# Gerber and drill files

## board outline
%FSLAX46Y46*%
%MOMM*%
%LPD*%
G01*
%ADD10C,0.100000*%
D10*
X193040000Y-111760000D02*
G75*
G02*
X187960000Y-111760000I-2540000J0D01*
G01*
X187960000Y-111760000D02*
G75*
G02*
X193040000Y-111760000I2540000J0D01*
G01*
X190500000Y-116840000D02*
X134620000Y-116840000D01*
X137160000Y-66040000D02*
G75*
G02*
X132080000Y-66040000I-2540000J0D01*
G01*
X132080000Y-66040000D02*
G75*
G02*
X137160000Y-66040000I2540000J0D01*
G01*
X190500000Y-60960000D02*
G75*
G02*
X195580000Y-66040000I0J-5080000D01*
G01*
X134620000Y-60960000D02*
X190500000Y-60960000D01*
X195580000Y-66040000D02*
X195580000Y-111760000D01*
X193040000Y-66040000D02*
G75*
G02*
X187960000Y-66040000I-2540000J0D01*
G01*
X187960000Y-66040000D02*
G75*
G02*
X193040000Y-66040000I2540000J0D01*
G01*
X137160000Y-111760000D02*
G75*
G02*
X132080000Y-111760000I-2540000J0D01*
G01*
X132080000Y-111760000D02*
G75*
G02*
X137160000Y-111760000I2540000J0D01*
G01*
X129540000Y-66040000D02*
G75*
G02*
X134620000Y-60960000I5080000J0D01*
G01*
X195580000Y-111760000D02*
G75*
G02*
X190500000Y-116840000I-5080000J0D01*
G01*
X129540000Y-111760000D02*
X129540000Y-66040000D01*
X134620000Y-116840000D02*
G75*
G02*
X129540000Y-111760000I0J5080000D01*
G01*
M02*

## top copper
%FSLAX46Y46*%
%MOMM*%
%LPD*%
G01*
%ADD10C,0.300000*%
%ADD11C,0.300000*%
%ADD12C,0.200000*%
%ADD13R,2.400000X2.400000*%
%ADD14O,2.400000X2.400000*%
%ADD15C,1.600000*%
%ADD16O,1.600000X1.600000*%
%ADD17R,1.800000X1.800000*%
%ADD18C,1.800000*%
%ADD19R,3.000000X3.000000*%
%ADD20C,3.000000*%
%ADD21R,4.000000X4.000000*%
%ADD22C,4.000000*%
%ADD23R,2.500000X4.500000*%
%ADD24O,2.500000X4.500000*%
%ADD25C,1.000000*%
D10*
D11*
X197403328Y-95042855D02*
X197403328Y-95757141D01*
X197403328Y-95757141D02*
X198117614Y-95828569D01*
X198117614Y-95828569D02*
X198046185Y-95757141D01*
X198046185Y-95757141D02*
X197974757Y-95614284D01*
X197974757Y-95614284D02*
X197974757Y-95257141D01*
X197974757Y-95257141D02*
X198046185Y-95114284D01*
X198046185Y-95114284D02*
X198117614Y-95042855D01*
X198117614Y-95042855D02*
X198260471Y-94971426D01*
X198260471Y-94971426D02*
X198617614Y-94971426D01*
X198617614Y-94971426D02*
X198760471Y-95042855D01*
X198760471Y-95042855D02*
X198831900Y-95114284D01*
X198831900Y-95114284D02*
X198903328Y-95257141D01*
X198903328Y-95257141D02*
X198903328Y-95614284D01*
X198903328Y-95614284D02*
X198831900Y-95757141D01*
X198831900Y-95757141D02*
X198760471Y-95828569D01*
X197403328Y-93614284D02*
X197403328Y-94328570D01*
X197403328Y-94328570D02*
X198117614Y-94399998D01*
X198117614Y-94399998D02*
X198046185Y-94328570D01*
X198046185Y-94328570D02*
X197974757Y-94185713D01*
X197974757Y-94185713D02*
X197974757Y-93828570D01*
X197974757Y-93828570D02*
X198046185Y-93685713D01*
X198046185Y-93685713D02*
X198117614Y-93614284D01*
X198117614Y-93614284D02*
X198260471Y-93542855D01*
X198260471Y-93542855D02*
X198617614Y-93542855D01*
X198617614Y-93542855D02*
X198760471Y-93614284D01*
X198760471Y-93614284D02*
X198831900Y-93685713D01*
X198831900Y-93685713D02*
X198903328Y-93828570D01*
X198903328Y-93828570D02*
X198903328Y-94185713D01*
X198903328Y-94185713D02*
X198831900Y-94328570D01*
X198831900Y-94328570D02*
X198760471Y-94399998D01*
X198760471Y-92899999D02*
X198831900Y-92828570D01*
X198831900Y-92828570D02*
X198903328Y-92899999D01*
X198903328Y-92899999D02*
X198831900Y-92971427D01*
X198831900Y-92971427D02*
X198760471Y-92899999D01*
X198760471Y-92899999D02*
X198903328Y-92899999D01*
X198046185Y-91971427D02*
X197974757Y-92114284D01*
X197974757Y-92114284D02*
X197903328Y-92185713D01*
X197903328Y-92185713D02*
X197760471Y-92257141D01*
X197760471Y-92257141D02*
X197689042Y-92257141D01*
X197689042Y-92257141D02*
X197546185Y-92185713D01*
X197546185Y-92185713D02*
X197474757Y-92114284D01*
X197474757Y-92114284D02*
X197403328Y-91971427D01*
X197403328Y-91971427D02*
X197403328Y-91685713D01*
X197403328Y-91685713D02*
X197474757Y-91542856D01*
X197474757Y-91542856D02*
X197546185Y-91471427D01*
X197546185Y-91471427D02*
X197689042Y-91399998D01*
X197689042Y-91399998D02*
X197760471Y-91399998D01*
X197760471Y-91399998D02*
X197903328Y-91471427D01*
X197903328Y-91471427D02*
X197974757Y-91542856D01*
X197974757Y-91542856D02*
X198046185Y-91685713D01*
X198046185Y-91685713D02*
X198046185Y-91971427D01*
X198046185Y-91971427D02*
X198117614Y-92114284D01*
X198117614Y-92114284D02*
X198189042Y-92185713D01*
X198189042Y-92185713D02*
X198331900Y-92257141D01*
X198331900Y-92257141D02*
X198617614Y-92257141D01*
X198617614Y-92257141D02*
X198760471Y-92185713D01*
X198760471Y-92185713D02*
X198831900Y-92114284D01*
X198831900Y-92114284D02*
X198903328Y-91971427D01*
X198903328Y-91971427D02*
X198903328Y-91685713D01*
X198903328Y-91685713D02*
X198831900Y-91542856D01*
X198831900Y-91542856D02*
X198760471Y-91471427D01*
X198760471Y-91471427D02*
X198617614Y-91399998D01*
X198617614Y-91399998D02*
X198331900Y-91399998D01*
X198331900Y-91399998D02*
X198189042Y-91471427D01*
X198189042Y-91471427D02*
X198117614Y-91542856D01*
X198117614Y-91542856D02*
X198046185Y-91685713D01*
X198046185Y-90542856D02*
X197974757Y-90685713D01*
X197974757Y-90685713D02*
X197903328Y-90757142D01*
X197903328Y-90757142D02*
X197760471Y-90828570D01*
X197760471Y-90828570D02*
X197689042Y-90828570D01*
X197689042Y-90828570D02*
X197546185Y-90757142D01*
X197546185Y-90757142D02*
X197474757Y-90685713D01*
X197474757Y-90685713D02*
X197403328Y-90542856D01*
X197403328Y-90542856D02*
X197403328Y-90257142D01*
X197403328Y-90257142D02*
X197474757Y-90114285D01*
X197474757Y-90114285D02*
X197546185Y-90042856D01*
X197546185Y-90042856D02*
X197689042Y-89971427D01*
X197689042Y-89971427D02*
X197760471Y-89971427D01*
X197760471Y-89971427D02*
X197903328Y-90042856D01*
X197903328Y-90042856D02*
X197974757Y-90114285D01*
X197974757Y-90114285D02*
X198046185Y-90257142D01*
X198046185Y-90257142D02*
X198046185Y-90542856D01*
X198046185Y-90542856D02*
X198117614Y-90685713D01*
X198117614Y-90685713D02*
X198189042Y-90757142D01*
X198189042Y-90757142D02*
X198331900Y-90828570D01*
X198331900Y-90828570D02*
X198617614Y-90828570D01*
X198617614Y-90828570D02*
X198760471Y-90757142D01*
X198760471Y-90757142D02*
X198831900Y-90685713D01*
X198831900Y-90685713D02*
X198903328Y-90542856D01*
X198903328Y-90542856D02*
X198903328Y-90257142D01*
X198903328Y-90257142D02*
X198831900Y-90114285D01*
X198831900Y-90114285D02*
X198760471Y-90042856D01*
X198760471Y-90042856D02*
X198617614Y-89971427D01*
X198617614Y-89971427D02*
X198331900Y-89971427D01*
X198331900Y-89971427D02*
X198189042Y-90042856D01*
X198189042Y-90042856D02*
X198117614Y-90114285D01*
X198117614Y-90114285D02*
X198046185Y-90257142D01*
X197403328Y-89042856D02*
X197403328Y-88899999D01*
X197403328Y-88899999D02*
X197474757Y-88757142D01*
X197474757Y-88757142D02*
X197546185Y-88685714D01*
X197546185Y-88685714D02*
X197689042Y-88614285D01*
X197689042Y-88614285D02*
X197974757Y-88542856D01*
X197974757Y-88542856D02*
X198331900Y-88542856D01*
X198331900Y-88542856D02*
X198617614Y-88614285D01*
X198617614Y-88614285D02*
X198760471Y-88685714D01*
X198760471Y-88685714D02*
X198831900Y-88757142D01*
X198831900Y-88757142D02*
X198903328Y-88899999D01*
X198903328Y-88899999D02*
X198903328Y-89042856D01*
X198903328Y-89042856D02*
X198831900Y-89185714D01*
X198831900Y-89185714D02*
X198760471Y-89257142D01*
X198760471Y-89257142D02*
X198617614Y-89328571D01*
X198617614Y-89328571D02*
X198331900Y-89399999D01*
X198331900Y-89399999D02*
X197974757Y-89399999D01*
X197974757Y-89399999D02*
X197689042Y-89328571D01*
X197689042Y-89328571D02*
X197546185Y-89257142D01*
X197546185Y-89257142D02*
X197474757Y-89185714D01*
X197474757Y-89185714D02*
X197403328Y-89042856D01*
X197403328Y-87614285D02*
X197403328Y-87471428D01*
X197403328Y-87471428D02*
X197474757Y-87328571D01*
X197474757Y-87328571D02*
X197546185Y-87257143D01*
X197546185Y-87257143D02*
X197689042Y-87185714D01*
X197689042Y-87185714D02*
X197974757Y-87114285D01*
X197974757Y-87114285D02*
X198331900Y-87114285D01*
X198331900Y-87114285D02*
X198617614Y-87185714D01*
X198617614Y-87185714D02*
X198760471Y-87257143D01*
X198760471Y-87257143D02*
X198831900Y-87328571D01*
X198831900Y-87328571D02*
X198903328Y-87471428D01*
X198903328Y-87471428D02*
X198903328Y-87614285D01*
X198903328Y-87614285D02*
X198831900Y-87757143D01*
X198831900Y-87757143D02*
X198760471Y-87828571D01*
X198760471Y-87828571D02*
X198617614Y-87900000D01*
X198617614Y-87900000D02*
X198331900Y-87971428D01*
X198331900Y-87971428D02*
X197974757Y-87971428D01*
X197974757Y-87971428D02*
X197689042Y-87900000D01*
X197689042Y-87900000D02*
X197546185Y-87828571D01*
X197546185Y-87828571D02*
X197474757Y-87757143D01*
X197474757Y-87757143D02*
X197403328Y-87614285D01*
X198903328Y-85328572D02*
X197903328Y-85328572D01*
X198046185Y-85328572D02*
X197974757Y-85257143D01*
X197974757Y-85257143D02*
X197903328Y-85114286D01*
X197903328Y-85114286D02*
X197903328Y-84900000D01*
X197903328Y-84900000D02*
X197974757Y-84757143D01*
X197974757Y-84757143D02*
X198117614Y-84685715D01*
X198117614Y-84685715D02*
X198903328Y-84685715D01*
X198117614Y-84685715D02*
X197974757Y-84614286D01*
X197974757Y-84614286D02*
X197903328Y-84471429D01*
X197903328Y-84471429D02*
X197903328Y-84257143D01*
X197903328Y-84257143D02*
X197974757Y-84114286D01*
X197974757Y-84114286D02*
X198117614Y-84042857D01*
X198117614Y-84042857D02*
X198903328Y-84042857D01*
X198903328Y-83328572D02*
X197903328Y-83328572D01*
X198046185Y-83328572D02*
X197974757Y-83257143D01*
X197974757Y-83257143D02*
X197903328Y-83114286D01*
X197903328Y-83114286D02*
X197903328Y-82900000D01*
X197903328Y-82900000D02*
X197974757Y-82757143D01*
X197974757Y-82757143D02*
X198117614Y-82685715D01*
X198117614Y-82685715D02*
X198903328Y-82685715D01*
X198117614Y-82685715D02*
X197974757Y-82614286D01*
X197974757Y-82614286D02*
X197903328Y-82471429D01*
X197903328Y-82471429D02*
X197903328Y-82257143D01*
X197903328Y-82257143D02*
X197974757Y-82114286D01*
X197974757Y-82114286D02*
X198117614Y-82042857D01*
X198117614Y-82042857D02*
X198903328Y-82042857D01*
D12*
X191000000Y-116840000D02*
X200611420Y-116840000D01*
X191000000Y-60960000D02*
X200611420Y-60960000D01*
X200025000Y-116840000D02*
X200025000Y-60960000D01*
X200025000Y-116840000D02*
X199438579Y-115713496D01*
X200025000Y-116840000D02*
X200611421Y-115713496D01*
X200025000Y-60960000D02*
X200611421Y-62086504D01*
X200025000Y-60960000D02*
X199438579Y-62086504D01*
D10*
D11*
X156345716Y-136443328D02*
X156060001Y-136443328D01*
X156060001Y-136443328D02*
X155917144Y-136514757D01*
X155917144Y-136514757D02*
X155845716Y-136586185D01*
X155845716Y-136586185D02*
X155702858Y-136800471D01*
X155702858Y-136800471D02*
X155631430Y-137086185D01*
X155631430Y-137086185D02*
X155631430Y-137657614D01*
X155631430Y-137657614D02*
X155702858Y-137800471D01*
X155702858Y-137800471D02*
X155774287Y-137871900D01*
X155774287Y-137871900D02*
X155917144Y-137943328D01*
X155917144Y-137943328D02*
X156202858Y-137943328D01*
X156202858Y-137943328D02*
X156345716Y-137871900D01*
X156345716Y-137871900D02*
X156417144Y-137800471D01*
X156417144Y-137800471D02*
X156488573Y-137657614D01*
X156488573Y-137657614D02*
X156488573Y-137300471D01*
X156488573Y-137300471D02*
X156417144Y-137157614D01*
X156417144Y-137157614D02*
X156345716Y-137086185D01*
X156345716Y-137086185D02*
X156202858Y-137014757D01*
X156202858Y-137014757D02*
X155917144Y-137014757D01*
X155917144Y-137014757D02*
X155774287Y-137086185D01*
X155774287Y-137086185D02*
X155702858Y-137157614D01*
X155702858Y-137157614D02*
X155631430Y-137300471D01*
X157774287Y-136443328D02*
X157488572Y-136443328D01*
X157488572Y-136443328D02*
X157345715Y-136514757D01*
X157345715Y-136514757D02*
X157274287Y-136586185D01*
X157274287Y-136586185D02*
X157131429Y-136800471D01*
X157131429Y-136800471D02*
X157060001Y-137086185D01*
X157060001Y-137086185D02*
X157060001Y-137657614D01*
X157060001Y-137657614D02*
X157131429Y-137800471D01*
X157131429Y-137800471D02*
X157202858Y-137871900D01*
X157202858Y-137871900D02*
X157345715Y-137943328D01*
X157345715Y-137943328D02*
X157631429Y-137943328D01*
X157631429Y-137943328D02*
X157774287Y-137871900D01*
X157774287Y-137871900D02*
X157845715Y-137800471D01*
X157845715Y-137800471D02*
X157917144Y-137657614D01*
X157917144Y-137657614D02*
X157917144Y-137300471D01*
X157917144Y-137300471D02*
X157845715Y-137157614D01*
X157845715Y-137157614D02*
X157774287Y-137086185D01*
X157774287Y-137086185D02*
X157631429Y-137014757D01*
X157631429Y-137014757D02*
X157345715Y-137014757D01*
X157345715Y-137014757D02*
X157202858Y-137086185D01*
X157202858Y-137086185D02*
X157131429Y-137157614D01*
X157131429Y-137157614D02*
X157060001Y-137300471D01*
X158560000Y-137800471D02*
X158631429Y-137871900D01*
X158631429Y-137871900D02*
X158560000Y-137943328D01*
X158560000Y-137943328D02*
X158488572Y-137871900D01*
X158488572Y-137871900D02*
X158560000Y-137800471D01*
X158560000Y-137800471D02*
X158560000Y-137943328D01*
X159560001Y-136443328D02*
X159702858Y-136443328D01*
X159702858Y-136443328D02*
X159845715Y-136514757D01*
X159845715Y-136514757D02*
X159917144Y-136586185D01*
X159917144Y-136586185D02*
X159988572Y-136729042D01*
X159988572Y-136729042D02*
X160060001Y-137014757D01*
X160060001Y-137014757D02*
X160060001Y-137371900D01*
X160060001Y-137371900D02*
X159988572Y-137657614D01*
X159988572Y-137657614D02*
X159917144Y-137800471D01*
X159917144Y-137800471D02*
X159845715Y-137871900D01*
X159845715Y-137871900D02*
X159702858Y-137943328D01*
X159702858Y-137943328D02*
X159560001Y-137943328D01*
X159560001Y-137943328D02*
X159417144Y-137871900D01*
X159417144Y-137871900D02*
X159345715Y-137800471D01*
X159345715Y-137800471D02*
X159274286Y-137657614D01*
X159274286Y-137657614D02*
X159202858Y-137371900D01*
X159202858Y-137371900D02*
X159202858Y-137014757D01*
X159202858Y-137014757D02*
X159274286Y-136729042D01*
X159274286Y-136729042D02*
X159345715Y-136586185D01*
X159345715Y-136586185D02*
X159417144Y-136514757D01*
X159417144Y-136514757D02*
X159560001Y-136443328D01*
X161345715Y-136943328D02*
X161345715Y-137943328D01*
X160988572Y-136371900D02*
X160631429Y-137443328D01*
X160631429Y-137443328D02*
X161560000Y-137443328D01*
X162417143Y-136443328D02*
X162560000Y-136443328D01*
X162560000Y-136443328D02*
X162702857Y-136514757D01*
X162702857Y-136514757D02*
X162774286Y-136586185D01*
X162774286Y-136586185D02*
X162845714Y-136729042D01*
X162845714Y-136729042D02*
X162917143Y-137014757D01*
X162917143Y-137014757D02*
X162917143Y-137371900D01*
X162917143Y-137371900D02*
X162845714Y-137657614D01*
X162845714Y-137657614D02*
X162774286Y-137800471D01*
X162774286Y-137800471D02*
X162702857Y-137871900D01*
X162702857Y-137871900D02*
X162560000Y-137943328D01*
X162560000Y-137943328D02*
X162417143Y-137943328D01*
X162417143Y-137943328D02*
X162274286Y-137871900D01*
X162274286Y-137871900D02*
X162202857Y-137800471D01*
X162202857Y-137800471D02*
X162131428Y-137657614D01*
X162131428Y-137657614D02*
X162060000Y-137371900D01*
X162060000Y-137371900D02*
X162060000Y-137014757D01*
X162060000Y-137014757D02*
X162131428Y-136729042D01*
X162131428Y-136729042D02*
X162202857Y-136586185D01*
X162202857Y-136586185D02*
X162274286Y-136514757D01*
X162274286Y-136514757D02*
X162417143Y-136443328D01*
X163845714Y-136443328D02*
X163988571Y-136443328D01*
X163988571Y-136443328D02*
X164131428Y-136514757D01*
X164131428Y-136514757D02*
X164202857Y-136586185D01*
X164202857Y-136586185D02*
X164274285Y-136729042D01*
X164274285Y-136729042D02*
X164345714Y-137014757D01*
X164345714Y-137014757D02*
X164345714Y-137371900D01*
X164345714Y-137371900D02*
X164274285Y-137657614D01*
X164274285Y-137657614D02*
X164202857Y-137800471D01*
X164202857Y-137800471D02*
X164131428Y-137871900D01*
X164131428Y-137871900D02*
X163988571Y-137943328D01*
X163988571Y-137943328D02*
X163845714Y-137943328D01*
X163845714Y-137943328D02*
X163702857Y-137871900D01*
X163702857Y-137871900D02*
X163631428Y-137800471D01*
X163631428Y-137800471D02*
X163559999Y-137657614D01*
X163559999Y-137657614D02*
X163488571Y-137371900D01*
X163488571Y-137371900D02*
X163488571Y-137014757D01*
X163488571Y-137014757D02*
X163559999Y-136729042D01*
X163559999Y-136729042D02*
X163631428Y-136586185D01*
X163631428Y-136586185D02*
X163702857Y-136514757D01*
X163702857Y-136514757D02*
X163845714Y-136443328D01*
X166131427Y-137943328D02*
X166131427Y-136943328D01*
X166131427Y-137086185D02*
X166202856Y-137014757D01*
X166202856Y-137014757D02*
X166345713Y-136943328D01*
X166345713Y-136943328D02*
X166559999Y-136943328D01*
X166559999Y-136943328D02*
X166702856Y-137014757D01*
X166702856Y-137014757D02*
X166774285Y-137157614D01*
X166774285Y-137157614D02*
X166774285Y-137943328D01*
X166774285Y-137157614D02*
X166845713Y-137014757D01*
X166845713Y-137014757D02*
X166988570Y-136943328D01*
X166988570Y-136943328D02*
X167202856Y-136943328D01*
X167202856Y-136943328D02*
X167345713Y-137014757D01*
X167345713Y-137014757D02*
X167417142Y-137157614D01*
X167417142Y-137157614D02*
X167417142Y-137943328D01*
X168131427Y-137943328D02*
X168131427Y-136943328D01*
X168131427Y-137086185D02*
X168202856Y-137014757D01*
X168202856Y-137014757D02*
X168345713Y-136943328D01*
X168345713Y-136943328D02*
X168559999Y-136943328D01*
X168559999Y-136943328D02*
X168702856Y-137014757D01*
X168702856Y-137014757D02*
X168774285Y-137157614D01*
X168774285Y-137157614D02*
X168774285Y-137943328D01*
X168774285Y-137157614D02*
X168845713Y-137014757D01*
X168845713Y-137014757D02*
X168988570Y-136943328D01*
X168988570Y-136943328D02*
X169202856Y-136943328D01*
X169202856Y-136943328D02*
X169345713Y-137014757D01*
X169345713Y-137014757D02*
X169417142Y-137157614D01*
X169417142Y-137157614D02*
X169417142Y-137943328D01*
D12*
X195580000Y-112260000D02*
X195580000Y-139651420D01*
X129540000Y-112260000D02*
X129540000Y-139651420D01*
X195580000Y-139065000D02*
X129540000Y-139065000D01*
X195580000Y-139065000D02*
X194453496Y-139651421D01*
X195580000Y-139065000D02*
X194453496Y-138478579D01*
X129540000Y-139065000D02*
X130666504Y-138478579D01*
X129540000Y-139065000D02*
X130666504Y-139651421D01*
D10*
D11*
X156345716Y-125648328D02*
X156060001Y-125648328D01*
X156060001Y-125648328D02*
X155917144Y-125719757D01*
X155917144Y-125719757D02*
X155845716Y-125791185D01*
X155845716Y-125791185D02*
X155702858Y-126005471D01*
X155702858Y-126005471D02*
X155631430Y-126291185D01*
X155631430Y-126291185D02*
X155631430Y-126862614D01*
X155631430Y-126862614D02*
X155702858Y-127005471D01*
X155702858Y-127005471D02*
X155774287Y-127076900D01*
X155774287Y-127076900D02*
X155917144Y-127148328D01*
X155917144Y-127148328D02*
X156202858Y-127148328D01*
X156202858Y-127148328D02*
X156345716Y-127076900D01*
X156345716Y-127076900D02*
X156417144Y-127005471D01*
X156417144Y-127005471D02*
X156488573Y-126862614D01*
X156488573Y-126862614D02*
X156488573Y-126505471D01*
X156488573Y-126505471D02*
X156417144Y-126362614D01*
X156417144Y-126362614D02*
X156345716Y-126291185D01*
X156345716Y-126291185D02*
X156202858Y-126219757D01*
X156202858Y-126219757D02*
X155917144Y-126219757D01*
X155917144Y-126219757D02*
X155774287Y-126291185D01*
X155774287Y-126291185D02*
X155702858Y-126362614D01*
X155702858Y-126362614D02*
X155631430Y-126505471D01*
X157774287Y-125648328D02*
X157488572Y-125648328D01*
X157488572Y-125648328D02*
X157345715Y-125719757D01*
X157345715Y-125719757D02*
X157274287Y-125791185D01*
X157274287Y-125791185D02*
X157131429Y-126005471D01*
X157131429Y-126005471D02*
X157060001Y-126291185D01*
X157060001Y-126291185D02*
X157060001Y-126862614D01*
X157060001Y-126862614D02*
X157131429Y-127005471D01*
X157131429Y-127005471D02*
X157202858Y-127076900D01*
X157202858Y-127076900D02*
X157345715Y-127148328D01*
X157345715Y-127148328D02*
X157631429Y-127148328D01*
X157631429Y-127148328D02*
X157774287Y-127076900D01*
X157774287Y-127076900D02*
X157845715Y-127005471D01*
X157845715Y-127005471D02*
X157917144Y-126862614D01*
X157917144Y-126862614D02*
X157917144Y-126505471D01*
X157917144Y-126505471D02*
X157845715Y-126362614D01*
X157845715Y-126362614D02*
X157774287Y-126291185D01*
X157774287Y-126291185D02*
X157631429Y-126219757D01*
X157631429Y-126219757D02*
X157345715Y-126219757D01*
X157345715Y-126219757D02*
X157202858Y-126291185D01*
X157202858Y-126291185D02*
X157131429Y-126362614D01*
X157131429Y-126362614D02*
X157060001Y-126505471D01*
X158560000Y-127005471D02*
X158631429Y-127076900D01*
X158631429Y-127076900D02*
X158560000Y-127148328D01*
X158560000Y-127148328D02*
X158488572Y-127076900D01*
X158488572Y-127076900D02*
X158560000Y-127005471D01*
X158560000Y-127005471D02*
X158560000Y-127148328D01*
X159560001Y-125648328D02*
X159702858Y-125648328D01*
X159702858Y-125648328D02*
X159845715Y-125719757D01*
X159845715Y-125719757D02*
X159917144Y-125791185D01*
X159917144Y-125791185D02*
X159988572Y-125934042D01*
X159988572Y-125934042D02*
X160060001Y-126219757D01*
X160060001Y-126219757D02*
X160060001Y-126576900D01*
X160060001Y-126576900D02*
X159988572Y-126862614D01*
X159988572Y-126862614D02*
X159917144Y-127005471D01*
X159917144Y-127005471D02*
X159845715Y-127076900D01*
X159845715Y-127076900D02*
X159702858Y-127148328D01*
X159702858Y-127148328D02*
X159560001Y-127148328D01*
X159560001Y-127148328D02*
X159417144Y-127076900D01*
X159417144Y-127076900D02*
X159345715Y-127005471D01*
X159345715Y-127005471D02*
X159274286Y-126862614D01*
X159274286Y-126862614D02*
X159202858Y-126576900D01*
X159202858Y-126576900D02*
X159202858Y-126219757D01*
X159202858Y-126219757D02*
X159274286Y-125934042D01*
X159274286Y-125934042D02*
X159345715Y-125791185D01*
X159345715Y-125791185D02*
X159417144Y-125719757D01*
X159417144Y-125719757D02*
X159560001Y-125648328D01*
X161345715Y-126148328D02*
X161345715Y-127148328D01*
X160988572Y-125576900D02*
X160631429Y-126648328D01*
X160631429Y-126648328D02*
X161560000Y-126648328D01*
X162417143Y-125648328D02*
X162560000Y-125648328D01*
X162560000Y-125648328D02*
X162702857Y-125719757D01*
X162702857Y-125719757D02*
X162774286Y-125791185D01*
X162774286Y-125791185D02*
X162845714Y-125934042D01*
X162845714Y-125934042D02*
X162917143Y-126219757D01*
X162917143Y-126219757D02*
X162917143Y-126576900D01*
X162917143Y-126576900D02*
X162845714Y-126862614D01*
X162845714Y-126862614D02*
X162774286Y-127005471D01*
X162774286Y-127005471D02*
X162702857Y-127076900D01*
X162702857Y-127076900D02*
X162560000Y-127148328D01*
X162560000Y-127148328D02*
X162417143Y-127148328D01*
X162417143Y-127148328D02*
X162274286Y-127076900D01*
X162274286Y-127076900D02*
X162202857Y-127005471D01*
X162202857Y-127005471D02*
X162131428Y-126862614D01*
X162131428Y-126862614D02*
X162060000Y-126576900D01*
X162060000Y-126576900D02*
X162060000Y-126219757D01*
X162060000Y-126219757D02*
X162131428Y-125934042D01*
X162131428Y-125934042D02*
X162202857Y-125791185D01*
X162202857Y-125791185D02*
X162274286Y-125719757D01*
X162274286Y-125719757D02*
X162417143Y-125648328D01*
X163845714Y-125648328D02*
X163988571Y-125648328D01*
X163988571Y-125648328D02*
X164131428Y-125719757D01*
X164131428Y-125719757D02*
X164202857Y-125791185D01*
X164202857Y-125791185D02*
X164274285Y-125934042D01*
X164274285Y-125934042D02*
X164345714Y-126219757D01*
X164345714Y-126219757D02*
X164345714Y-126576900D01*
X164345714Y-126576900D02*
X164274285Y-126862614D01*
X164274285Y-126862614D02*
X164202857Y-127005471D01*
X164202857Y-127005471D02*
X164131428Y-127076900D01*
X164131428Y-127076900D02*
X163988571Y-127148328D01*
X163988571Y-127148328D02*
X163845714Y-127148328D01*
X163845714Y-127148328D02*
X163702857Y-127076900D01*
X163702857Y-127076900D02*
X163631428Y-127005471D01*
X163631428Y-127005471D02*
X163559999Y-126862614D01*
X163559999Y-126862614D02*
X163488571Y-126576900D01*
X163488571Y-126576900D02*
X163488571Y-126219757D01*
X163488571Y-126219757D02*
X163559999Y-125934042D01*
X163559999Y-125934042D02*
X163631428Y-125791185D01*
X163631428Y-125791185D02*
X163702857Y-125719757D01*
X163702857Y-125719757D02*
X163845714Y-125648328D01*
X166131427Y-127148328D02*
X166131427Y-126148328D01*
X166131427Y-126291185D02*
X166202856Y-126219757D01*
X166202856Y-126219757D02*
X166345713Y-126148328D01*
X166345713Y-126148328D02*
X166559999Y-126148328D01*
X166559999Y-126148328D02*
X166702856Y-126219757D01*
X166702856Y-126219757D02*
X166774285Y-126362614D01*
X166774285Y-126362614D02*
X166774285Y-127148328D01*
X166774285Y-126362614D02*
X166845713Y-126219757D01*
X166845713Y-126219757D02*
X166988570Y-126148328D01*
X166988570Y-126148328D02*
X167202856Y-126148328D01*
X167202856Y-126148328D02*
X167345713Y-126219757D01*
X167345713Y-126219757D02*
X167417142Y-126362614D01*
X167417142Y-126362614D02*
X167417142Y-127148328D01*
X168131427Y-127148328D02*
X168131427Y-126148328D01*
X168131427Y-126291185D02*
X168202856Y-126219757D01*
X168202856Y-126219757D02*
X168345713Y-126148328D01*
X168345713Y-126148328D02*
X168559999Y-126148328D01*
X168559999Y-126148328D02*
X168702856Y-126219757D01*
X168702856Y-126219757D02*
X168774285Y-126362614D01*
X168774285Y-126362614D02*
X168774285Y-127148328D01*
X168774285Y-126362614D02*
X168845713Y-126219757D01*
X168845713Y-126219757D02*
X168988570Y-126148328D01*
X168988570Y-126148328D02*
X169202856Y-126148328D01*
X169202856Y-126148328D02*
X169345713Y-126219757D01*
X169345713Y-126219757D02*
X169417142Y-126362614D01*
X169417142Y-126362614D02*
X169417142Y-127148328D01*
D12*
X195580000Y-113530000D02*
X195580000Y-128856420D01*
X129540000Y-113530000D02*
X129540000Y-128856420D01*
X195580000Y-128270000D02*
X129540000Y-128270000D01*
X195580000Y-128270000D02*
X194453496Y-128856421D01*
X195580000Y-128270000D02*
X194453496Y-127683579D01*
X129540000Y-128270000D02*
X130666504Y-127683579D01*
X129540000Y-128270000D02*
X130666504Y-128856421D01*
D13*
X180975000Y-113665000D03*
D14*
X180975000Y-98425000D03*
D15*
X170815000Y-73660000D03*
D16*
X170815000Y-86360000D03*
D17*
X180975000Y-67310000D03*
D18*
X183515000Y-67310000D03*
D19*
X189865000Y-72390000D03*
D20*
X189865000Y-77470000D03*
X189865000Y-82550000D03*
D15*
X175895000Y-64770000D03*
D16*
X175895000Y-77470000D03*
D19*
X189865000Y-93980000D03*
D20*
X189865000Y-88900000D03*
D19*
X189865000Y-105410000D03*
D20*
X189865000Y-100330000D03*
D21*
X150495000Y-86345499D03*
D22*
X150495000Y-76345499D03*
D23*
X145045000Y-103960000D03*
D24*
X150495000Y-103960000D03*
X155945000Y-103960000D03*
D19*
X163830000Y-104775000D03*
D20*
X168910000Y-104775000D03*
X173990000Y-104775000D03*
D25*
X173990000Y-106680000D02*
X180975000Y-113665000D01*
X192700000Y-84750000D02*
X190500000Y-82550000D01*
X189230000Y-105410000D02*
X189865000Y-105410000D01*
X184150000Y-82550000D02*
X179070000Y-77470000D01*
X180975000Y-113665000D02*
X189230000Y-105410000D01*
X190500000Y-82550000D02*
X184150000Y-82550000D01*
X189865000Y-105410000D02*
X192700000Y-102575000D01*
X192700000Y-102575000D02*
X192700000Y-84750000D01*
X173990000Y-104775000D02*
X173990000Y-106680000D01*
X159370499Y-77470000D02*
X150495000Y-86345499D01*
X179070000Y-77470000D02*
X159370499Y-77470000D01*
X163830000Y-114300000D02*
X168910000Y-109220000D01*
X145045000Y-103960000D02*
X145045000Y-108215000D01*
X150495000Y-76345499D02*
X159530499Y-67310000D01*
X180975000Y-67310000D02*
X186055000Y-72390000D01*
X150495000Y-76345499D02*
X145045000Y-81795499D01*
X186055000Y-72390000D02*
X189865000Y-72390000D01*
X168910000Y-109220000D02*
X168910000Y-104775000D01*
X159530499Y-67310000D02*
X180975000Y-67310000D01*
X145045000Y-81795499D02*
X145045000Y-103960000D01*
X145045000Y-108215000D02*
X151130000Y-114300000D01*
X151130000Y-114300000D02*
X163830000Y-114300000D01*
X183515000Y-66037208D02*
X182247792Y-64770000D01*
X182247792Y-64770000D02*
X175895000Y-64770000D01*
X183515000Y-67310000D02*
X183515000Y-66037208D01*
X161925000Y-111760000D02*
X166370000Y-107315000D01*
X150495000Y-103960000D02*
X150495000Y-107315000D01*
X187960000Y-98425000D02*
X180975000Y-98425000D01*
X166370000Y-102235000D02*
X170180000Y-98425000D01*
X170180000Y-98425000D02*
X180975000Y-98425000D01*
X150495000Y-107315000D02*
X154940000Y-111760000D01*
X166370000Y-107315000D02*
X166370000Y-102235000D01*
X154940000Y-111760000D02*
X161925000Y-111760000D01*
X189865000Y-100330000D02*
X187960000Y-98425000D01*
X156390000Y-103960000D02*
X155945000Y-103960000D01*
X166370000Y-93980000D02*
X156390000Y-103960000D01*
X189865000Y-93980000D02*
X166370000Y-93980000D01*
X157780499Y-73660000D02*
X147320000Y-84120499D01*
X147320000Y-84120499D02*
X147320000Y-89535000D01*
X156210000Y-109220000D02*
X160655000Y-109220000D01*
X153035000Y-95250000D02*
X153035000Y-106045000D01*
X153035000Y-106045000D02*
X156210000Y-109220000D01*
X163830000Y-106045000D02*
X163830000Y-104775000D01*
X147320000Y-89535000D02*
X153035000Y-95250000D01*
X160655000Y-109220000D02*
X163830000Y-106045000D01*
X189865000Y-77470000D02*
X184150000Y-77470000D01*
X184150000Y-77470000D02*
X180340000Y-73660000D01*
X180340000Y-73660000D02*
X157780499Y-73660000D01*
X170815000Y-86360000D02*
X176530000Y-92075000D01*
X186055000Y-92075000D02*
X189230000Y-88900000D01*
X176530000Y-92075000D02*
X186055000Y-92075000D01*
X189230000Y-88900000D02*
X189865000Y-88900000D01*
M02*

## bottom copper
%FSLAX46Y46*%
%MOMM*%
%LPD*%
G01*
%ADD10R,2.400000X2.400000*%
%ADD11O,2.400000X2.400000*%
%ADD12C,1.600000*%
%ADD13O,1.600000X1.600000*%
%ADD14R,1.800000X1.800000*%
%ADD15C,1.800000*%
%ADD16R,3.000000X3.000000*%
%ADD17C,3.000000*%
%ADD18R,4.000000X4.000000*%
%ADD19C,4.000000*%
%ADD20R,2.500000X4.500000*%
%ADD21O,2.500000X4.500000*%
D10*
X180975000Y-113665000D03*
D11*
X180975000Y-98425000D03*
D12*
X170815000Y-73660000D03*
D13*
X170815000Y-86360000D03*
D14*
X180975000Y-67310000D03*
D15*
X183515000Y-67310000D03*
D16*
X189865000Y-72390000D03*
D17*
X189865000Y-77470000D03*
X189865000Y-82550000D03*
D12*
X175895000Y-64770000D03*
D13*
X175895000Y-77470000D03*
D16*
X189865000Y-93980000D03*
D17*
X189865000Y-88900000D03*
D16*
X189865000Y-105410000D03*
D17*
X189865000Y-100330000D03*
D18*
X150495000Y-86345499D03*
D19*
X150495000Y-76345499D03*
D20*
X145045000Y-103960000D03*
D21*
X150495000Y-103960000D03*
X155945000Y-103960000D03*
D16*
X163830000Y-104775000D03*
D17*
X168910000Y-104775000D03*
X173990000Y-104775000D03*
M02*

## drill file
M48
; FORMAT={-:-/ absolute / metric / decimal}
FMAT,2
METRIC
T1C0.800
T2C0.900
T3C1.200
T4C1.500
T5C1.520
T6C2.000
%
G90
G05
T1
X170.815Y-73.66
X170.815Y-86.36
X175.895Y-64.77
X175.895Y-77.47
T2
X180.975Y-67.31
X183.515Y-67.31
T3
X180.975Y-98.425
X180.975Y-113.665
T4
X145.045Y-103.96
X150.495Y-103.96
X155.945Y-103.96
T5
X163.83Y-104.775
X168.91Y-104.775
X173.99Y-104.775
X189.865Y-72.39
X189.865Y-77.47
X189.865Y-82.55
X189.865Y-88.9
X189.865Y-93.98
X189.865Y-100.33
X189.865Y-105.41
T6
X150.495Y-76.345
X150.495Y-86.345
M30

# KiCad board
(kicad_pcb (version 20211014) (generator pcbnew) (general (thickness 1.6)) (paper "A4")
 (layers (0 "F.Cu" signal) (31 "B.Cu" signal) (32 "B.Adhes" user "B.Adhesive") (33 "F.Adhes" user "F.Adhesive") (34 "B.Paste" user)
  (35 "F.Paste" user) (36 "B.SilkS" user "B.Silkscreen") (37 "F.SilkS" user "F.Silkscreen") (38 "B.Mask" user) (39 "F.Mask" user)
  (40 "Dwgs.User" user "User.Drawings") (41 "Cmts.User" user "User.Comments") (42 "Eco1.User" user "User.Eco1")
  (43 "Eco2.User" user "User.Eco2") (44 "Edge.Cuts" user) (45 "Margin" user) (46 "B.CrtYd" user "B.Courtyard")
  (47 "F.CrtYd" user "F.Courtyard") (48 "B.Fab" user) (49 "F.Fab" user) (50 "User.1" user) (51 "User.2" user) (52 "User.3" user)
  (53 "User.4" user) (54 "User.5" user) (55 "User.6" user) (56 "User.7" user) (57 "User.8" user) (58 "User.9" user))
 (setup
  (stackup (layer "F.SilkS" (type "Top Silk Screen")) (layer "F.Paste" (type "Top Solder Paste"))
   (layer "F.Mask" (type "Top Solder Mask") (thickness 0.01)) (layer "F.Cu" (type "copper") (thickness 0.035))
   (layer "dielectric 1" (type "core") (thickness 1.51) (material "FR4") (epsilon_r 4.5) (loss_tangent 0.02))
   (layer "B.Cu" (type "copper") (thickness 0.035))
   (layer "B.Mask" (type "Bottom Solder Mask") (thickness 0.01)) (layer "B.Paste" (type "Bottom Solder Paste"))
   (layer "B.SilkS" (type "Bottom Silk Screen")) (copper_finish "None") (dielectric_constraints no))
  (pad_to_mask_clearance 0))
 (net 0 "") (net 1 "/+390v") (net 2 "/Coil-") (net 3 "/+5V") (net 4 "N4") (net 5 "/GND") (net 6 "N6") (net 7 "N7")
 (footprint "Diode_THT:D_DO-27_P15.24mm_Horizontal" (layer "F.Cu") (at 180.975 113.665 90)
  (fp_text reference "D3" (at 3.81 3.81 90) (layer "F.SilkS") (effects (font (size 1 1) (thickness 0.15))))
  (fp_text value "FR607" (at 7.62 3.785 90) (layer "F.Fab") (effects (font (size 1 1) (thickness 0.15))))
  (pad "1" thru_hole rect (at 0 0 90) (size 2.4 2.4) (drill 1.2) (layers *.Cu *.Mask) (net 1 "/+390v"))
  (pad "2" thru_hole oval (at 15.24 0 90) (size 2.4 2.4) (drill 1.2) (layers *.Cu *.Mask) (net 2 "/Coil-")))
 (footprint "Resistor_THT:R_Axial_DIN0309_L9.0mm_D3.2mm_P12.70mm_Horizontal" (layer "F.Cu") (at 170.815 73.66 -90)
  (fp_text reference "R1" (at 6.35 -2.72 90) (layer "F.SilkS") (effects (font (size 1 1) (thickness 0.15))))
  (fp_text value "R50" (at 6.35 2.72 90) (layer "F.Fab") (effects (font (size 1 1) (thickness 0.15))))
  (pad "1" thru_hole circle (at 0 0 270) (size 1.6 1.6) (drill 0.8) (layers *.Cu *.Mask) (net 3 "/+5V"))
  (pad "2" thru_hole oval (at 12.7 0 270) (size 1.6 1.6) (drill 0.8) (layers *.Cu *.Mask) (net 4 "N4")))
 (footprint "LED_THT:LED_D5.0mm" (layer "F.Cu") (at 180.975 67.31)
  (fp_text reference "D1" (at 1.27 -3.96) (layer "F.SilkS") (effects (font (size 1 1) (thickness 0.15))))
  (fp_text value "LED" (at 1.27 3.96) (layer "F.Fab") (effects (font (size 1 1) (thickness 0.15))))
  (pad "1" thru_hole rect (at 0 0) (size 1.8 1.8) (drill 0.9) (layers *.Cu *.Mask) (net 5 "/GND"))
  (pad "2" thru_hole circle (at 2.54 0) (size 1.8 1.8) (drill 0.9) (layers *.Cu *.Mask) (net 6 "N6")))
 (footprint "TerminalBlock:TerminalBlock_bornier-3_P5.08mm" (layer "F.Cu") (at 189.865 72.39 -90)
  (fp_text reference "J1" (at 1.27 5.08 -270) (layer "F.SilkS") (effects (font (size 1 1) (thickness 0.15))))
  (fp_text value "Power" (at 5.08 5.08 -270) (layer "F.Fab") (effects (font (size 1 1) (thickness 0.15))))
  (pad "1" thru_hole rect (at 0 0 270) (size 3 3) (drill 1.52) (layers *.Cu *.Mask) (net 5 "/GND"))
  (pad "2" thru_hole circle (at 5.08 0 270) (size 3 3) (drill 1.52) (layers *.Cu *.Mask) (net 3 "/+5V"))
  (pad "3" thru_hole circle (at 10.16 0 270) (size 3 3) (drill 1.52) (layers *.Cu *.Mask) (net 1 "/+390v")))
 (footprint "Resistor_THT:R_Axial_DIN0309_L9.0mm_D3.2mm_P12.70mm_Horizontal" (layer "F.Cu") (at 175.895 64.77 -90)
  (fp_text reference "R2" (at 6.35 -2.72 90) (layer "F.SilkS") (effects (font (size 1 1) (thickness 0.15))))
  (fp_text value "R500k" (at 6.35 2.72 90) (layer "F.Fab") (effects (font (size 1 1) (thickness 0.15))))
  (pad "1" thru_hole circle (at 0 0 270) (size 1.6 1.6) (drill 0.8) (layers *.Cu *.Mask) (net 6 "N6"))
  (pad "2" thru_hole oval (at 12.7 0 270) (size 1.6 1.6) (drill 0.8) (layers *.Cu *.Mask) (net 1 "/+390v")))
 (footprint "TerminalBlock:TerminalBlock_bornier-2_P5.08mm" (layer "F.Cu") (at 189.865 93.98 90)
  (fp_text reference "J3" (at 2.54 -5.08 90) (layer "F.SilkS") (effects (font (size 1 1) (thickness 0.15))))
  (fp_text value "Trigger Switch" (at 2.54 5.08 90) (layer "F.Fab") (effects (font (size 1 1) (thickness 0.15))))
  (pad "1" thru_hole rect (at 0 0 90) (size 3 3) (drill 1.52) (layers *.Cu *.Mask) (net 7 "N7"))
  (pad "2" thru_hole circle (at 5.08 0 90) (size 3 3) (drill 1.52) (layers *.Cu *.Mask) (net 4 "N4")))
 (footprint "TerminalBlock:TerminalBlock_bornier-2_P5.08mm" (layer "F.Cu") (at 189.865 105.41 90)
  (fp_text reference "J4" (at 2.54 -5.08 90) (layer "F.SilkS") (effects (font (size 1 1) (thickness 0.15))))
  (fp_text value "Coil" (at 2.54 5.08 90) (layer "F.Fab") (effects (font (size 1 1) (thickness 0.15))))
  (pad "1" thru_hole rect (at 0 0 90) (size 3 3) (drill 1.52) (layers *.Cu *.Mask) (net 1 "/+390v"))
  (pad "2" thru_hole circle (at 5.08 0 90) (size 3 3) (drill 1.52) (layers *.Cu *.Mask) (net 2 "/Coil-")))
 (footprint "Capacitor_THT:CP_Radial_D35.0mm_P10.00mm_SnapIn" (layer "F.Cu") (at 150.495 86.345499 90)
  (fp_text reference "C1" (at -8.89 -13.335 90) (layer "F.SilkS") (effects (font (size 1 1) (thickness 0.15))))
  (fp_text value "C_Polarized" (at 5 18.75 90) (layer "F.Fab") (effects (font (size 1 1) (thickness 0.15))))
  (pad "1" thru_hole rect (at 0 0 90) (size 4 4) (drill 2) (layers *.Cu *.Mask) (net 1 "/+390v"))
  (pad "2" thru_hole circle (at 10 0 90) (size 4 4) (drill 2) (layers *.Cu *.Mask) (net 5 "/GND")))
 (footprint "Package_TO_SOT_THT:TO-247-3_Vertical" (layer "F.Cu") (at 145.045 103.96)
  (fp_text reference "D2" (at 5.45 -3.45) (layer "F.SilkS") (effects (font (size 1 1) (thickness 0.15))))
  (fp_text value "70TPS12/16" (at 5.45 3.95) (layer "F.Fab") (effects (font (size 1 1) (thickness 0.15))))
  (pad "1" thru_hole rect (at 0 0) (size 2.5 4.5) (drill 1.5) (layers *.Cu *.Mask) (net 5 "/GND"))
  (pad "2" thru_hole oval (at 5.45 0) (size 2.5 4.5) (drill 1.5) (layers *.Cu *.Mask) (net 2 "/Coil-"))
  (pad "3" thru_hole oval (at 10.9 0) (size 2.5 4.5) (drill 1.5) (layers *.Cu *.Mask) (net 7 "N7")))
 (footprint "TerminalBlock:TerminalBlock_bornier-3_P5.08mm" (layer "F.Cu") (at 163.83 104.775)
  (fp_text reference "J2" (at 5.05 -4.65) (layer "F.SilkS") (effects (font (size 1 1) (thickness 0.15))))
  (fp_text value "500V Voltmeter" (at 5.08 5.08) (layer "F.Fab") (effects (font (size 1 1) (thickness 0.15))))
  (pad "1" thru_hole rect (at 0 0) (size 3 3) (drill 1.52) (layers *.Cu *.Mask) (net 3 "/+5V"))
  (pad "2" thru_hole circle (at 5.08 0) (size 3 3) (drill 1.52) (layers *.Cu *.Mask) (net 5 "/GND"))
  (pad "3" thru_hole circle (at 10.16 0) (size 3 3) (drill 1.52) (layers *.Cu *.Mask) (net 1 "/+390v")))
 (gr_circle (center 190.5 111.76) (end 193.04 111.76) (layer "Edge.Cuts") (width 0.1) (fill none))
 (gr_line (start 190.5 116.84) (end 134.62 116.84) (layer "Edge.Cuts") (width 0.1))
 (gr_circle (center 134.62 66.04) (end 137.16 66.04) (layer "Edge.Cuts") (width 0.1) (fill none))
 (gr_arc (start 190.5 60.96) (mid 194.092102 62.447898) (end 195.58 66.04) (layer "Edge.Cuts") (width 0.1))
 (gr_line (start 134.62 60.96) (end 190.5 60.96) (layer "Edge.Cuts") (width 0.1))
 (gr_line (start 195.58 66.04) (end 195.58 111.76) (layer "Edge.Cuts") (width 0.1))
 (gr_circle (center 190.5 66.04) (end 193.04 66.04) (layer "Edge.Cuts") (width 0.1) (fill none))
 (gr_circle (center 134.62 111.76) (end 137.16 111.76) (layer "Edge.Cuts") (width 0.1) (fill none))
 (gr_arc (start 129.54 66.04) (mid 131.027898 62.447898) (end 134.62 60.96) (layer "Edge.Cuts") (width 0.1))
 (gr_arc (start 195.58 111.76) (mid 194.092102 115.352102) (end 190.5 116.84) (layer "Edge.Cuts") (width 0.1))
 (gr_line (start 129.54 111.76) (end 129.54 66.04) (layer "Edge.Cuts") (width 0.1))
 (gr_arc (start 134.62 116.84) (mid 131.027898 115.352102) (end 129.54 111.76) (layer "Edge.Cuts") (width 0.1))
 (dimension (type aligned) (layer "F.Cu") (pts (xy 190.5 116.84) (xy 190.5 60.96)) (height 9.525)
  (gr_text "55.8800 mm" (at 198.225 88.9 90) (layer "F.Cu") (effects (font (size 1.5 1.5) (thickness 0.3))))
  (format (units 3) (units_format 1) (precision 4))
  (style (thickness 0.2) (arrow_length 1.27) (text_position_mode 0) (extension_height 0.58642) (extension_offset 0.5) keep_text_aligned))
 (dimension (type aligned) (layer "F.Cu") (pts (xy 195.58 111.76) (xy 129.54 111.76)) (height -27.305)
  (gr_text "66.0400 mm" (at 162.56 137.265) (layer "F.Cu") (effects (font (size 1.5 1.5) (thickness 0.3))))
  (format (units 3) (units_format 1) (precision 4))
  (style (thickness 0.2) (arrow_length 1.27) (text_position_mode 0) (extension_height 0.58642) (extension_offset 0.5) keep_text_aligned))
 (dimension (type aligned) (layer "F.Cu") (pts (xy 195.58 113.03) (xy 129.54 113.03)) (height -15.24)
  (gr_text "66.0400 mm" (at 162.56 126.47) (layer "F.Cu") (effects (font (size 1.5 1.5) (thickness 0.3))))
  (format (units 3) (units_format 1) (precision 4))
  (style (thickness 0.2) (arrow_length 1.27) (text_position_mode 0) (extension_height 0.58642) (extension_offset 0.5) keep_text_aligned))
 (segment (start 173.99 106.68) (end 180.975 113.665) (width 1) (layer "F.Cu") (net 1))
 (segment (start 192.7 84.75) (end 190.5 82.55) (width 1) (layer "F.Cu") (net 1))
 (segment (start 189.23 105.41) (end 189.865 105.41) (width 1) (layer "F.Cu") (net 1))
 (segment (start 184.15 82.55) (end 179.07 77.47) (width 1) (layer "F.Cu") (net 1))
 (segment (start 180.975 113.665) (end 189.23 105.41) (width 1) (layer "F.Cu") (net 1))
 (segment (start 190.5 82.55) (end 184.15 82.55) (width 1) (layer "F.Cu") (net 1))
 (segment (start 189.865 105.41) (end 192.7 102.575) (width 1) (layer "F.Cu") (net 1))
 (segment (start 192.7 102.575) (end 192.7 84.75) (width 1) (layer "F.Cu") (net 1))
 (segment (start 173.99 104.775) (end 173.99 106.68) (width 1) (layer "F.Cu") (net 1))
 (segment (start 159.370499 77.47) (end 150.495 86.345499) (width 1) (layer "F.Cu") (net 1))
 (segment (start 179.07 77.47) (end 159.370499 77.47) (width 1) (layer "F.Cu") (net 1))
 (segment (start 163.83 114.3) (end 168.91 109.22) (width 1) (layer "F.Cu") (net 5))
 (segment (start 145.045 103.96) (end 145.045 108.215) (width 1) (layer "F.Cu") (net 5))
 (segment (start 150.495 76.345499) (end 159.530499 67.31) (width 1) (layer "F.Cu") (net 5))
 (segment (start 180.975 67.31) (end 186.055 72.39) (width 1) (layer "F.Cu") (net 5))
 (segment (start 150.495 76.345499) (end 145.045 81.795499) (width 1) (layer "F.Cu") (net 5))
 (segment (start 186.055 72.39) (end 189.865 72.39) (width 1) (layer "F.Cu") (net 5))
 (segment (start 168.91 109.22) (end 168.91 104.775) (width 1) (layer "F.Cu") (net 5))
 (segment (start 159.530499 67.31) (end 180.975 67.31) (width 1) (layer "F.Cu") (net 5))
 (segment (start 145.045 81.795499) (end 145.045 103.96) (width 1) (layer "F.Cu") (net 5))
 (segment (start 145.045 108.215) (end 151.13 114.3) (width 1) (layer "F.Cu") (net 5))
 (segment (start 151.13 114.3) (end 163.83 114.3) (width 1) (layer "F.Cu") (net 5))
 (segment (start 183.515 66.037208) (end 182.247792 64.77) (width 1) (layer "F.Cu") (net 6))
 (segment (start 182.247792 64.77) (end 175.895 64.77) (width 1) (layer "F.Cu") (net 6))
 (segment (start 183.515 67.31) (end 183.515 66.037208) (width 1) (layer "F.Cu") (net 6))
 (segment (start 161.925 111.76) (end 166.37 107.315) (width 1) (layer "F.Cu") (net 2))
 (segment (start 150.495 103.96) (end 150.495 107.315) (width 1) (layer "F.Cu") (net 2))
 (segment (start 187.96 98.425) (end 180.975 98.425) (width 1) (layer "F.Cu") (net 2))
 (segment (start 166.37 102.235) (end 170.18 98.425) (width 1) (layer "F.Cu") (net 2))
 (segment (start 170.18 98.425) (end 180.975 98.425) (width 1) (layer "F.Cu") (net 2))
 (segment (start 150.495 107.315) (end 154.94 111.76) (width 1) (layer "F.Cu") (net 2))
 (segment (start 166.37 107.315) (end 166.37 102.235) (width 1) (layer "F.Cu") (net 2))
 (segment (start 154.94 111.76) (end 161.925 111.76) (width 1) (layer "F.Cu") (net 2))
 (segment (start 189.865 100.33) (end 187.96 98.425) (width 1) (layer "F.Cu") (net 2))
 (segment (start 156.39 103.96) (end 155.945 103.96) (width 1) (layer "F.Cu") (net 7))
 (segment (start 166.37 93.98) (end 156.39 103.96) (width 1) (layer "F.Cu") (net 7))
 (segment (start 189.865 93.98) (end 166.37 93.98) (width 1) (layer "F.Cu") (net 7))
 (segment (start 157.780499 73.66) (end 147.32 84.120499) (width 1) (layer "F.Cu") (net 3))
 (segment (start 147.32 84.120499) (end 147.32 89.535) (width 1) (layer "F.Cu") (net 3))
 (segment (start 156.21 109.22) (end 160.655 109.22) (width 1) (layer "F.Cu") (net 3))
 (segment (start 153.035 95.25) (end 153.035 106.045) (width 1) (layer "F.Cu") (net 3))
 (segment (start 153.035 106.045) (end 156.21 109.22) (width 1) (layer "F.Cu") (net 3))
 (segment (start 163.83 106.045) (end 163.83 104.775) (width 1) (layer "F.Cu") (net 3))
 (segment (start 147.32 89.535) (end 153.035 95.25) (width 1) (layer "F.Cu") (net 3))
 (segment (start 160.655 109.22) (end 163.83 106.045) (width 1) (layer "F.Cu") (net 3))
 (segment (start 189.865 77.47) (end 184.15 77.47) (width 1) (layer "F.Cu") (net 3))
 (segment (start 184.15 77.47) (end 180.34 73.66) (width 1) (layer "F.Cu") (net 3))
 (segment (start 180.34 73.66) (end 157.780499 73.66) (width 1) (layer "F.Cu") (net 3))
 (segment (start 170.815 86.36) (end 176.53 92.075) (width 1) (layer "F.Cu") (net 4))
 (segment (start 186.055 92.075) (end 189.23 88.9) (width 1) (layer "F.Cu") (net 4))
 (segment (start 176.53 92.075) (end 186.055 92.075) (width 1) (layer "F.Cu") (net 4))
 (segment (start 189.23 88.9) (end 189.865 88.9) (width 1) (layer "F.Cu") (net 4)))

